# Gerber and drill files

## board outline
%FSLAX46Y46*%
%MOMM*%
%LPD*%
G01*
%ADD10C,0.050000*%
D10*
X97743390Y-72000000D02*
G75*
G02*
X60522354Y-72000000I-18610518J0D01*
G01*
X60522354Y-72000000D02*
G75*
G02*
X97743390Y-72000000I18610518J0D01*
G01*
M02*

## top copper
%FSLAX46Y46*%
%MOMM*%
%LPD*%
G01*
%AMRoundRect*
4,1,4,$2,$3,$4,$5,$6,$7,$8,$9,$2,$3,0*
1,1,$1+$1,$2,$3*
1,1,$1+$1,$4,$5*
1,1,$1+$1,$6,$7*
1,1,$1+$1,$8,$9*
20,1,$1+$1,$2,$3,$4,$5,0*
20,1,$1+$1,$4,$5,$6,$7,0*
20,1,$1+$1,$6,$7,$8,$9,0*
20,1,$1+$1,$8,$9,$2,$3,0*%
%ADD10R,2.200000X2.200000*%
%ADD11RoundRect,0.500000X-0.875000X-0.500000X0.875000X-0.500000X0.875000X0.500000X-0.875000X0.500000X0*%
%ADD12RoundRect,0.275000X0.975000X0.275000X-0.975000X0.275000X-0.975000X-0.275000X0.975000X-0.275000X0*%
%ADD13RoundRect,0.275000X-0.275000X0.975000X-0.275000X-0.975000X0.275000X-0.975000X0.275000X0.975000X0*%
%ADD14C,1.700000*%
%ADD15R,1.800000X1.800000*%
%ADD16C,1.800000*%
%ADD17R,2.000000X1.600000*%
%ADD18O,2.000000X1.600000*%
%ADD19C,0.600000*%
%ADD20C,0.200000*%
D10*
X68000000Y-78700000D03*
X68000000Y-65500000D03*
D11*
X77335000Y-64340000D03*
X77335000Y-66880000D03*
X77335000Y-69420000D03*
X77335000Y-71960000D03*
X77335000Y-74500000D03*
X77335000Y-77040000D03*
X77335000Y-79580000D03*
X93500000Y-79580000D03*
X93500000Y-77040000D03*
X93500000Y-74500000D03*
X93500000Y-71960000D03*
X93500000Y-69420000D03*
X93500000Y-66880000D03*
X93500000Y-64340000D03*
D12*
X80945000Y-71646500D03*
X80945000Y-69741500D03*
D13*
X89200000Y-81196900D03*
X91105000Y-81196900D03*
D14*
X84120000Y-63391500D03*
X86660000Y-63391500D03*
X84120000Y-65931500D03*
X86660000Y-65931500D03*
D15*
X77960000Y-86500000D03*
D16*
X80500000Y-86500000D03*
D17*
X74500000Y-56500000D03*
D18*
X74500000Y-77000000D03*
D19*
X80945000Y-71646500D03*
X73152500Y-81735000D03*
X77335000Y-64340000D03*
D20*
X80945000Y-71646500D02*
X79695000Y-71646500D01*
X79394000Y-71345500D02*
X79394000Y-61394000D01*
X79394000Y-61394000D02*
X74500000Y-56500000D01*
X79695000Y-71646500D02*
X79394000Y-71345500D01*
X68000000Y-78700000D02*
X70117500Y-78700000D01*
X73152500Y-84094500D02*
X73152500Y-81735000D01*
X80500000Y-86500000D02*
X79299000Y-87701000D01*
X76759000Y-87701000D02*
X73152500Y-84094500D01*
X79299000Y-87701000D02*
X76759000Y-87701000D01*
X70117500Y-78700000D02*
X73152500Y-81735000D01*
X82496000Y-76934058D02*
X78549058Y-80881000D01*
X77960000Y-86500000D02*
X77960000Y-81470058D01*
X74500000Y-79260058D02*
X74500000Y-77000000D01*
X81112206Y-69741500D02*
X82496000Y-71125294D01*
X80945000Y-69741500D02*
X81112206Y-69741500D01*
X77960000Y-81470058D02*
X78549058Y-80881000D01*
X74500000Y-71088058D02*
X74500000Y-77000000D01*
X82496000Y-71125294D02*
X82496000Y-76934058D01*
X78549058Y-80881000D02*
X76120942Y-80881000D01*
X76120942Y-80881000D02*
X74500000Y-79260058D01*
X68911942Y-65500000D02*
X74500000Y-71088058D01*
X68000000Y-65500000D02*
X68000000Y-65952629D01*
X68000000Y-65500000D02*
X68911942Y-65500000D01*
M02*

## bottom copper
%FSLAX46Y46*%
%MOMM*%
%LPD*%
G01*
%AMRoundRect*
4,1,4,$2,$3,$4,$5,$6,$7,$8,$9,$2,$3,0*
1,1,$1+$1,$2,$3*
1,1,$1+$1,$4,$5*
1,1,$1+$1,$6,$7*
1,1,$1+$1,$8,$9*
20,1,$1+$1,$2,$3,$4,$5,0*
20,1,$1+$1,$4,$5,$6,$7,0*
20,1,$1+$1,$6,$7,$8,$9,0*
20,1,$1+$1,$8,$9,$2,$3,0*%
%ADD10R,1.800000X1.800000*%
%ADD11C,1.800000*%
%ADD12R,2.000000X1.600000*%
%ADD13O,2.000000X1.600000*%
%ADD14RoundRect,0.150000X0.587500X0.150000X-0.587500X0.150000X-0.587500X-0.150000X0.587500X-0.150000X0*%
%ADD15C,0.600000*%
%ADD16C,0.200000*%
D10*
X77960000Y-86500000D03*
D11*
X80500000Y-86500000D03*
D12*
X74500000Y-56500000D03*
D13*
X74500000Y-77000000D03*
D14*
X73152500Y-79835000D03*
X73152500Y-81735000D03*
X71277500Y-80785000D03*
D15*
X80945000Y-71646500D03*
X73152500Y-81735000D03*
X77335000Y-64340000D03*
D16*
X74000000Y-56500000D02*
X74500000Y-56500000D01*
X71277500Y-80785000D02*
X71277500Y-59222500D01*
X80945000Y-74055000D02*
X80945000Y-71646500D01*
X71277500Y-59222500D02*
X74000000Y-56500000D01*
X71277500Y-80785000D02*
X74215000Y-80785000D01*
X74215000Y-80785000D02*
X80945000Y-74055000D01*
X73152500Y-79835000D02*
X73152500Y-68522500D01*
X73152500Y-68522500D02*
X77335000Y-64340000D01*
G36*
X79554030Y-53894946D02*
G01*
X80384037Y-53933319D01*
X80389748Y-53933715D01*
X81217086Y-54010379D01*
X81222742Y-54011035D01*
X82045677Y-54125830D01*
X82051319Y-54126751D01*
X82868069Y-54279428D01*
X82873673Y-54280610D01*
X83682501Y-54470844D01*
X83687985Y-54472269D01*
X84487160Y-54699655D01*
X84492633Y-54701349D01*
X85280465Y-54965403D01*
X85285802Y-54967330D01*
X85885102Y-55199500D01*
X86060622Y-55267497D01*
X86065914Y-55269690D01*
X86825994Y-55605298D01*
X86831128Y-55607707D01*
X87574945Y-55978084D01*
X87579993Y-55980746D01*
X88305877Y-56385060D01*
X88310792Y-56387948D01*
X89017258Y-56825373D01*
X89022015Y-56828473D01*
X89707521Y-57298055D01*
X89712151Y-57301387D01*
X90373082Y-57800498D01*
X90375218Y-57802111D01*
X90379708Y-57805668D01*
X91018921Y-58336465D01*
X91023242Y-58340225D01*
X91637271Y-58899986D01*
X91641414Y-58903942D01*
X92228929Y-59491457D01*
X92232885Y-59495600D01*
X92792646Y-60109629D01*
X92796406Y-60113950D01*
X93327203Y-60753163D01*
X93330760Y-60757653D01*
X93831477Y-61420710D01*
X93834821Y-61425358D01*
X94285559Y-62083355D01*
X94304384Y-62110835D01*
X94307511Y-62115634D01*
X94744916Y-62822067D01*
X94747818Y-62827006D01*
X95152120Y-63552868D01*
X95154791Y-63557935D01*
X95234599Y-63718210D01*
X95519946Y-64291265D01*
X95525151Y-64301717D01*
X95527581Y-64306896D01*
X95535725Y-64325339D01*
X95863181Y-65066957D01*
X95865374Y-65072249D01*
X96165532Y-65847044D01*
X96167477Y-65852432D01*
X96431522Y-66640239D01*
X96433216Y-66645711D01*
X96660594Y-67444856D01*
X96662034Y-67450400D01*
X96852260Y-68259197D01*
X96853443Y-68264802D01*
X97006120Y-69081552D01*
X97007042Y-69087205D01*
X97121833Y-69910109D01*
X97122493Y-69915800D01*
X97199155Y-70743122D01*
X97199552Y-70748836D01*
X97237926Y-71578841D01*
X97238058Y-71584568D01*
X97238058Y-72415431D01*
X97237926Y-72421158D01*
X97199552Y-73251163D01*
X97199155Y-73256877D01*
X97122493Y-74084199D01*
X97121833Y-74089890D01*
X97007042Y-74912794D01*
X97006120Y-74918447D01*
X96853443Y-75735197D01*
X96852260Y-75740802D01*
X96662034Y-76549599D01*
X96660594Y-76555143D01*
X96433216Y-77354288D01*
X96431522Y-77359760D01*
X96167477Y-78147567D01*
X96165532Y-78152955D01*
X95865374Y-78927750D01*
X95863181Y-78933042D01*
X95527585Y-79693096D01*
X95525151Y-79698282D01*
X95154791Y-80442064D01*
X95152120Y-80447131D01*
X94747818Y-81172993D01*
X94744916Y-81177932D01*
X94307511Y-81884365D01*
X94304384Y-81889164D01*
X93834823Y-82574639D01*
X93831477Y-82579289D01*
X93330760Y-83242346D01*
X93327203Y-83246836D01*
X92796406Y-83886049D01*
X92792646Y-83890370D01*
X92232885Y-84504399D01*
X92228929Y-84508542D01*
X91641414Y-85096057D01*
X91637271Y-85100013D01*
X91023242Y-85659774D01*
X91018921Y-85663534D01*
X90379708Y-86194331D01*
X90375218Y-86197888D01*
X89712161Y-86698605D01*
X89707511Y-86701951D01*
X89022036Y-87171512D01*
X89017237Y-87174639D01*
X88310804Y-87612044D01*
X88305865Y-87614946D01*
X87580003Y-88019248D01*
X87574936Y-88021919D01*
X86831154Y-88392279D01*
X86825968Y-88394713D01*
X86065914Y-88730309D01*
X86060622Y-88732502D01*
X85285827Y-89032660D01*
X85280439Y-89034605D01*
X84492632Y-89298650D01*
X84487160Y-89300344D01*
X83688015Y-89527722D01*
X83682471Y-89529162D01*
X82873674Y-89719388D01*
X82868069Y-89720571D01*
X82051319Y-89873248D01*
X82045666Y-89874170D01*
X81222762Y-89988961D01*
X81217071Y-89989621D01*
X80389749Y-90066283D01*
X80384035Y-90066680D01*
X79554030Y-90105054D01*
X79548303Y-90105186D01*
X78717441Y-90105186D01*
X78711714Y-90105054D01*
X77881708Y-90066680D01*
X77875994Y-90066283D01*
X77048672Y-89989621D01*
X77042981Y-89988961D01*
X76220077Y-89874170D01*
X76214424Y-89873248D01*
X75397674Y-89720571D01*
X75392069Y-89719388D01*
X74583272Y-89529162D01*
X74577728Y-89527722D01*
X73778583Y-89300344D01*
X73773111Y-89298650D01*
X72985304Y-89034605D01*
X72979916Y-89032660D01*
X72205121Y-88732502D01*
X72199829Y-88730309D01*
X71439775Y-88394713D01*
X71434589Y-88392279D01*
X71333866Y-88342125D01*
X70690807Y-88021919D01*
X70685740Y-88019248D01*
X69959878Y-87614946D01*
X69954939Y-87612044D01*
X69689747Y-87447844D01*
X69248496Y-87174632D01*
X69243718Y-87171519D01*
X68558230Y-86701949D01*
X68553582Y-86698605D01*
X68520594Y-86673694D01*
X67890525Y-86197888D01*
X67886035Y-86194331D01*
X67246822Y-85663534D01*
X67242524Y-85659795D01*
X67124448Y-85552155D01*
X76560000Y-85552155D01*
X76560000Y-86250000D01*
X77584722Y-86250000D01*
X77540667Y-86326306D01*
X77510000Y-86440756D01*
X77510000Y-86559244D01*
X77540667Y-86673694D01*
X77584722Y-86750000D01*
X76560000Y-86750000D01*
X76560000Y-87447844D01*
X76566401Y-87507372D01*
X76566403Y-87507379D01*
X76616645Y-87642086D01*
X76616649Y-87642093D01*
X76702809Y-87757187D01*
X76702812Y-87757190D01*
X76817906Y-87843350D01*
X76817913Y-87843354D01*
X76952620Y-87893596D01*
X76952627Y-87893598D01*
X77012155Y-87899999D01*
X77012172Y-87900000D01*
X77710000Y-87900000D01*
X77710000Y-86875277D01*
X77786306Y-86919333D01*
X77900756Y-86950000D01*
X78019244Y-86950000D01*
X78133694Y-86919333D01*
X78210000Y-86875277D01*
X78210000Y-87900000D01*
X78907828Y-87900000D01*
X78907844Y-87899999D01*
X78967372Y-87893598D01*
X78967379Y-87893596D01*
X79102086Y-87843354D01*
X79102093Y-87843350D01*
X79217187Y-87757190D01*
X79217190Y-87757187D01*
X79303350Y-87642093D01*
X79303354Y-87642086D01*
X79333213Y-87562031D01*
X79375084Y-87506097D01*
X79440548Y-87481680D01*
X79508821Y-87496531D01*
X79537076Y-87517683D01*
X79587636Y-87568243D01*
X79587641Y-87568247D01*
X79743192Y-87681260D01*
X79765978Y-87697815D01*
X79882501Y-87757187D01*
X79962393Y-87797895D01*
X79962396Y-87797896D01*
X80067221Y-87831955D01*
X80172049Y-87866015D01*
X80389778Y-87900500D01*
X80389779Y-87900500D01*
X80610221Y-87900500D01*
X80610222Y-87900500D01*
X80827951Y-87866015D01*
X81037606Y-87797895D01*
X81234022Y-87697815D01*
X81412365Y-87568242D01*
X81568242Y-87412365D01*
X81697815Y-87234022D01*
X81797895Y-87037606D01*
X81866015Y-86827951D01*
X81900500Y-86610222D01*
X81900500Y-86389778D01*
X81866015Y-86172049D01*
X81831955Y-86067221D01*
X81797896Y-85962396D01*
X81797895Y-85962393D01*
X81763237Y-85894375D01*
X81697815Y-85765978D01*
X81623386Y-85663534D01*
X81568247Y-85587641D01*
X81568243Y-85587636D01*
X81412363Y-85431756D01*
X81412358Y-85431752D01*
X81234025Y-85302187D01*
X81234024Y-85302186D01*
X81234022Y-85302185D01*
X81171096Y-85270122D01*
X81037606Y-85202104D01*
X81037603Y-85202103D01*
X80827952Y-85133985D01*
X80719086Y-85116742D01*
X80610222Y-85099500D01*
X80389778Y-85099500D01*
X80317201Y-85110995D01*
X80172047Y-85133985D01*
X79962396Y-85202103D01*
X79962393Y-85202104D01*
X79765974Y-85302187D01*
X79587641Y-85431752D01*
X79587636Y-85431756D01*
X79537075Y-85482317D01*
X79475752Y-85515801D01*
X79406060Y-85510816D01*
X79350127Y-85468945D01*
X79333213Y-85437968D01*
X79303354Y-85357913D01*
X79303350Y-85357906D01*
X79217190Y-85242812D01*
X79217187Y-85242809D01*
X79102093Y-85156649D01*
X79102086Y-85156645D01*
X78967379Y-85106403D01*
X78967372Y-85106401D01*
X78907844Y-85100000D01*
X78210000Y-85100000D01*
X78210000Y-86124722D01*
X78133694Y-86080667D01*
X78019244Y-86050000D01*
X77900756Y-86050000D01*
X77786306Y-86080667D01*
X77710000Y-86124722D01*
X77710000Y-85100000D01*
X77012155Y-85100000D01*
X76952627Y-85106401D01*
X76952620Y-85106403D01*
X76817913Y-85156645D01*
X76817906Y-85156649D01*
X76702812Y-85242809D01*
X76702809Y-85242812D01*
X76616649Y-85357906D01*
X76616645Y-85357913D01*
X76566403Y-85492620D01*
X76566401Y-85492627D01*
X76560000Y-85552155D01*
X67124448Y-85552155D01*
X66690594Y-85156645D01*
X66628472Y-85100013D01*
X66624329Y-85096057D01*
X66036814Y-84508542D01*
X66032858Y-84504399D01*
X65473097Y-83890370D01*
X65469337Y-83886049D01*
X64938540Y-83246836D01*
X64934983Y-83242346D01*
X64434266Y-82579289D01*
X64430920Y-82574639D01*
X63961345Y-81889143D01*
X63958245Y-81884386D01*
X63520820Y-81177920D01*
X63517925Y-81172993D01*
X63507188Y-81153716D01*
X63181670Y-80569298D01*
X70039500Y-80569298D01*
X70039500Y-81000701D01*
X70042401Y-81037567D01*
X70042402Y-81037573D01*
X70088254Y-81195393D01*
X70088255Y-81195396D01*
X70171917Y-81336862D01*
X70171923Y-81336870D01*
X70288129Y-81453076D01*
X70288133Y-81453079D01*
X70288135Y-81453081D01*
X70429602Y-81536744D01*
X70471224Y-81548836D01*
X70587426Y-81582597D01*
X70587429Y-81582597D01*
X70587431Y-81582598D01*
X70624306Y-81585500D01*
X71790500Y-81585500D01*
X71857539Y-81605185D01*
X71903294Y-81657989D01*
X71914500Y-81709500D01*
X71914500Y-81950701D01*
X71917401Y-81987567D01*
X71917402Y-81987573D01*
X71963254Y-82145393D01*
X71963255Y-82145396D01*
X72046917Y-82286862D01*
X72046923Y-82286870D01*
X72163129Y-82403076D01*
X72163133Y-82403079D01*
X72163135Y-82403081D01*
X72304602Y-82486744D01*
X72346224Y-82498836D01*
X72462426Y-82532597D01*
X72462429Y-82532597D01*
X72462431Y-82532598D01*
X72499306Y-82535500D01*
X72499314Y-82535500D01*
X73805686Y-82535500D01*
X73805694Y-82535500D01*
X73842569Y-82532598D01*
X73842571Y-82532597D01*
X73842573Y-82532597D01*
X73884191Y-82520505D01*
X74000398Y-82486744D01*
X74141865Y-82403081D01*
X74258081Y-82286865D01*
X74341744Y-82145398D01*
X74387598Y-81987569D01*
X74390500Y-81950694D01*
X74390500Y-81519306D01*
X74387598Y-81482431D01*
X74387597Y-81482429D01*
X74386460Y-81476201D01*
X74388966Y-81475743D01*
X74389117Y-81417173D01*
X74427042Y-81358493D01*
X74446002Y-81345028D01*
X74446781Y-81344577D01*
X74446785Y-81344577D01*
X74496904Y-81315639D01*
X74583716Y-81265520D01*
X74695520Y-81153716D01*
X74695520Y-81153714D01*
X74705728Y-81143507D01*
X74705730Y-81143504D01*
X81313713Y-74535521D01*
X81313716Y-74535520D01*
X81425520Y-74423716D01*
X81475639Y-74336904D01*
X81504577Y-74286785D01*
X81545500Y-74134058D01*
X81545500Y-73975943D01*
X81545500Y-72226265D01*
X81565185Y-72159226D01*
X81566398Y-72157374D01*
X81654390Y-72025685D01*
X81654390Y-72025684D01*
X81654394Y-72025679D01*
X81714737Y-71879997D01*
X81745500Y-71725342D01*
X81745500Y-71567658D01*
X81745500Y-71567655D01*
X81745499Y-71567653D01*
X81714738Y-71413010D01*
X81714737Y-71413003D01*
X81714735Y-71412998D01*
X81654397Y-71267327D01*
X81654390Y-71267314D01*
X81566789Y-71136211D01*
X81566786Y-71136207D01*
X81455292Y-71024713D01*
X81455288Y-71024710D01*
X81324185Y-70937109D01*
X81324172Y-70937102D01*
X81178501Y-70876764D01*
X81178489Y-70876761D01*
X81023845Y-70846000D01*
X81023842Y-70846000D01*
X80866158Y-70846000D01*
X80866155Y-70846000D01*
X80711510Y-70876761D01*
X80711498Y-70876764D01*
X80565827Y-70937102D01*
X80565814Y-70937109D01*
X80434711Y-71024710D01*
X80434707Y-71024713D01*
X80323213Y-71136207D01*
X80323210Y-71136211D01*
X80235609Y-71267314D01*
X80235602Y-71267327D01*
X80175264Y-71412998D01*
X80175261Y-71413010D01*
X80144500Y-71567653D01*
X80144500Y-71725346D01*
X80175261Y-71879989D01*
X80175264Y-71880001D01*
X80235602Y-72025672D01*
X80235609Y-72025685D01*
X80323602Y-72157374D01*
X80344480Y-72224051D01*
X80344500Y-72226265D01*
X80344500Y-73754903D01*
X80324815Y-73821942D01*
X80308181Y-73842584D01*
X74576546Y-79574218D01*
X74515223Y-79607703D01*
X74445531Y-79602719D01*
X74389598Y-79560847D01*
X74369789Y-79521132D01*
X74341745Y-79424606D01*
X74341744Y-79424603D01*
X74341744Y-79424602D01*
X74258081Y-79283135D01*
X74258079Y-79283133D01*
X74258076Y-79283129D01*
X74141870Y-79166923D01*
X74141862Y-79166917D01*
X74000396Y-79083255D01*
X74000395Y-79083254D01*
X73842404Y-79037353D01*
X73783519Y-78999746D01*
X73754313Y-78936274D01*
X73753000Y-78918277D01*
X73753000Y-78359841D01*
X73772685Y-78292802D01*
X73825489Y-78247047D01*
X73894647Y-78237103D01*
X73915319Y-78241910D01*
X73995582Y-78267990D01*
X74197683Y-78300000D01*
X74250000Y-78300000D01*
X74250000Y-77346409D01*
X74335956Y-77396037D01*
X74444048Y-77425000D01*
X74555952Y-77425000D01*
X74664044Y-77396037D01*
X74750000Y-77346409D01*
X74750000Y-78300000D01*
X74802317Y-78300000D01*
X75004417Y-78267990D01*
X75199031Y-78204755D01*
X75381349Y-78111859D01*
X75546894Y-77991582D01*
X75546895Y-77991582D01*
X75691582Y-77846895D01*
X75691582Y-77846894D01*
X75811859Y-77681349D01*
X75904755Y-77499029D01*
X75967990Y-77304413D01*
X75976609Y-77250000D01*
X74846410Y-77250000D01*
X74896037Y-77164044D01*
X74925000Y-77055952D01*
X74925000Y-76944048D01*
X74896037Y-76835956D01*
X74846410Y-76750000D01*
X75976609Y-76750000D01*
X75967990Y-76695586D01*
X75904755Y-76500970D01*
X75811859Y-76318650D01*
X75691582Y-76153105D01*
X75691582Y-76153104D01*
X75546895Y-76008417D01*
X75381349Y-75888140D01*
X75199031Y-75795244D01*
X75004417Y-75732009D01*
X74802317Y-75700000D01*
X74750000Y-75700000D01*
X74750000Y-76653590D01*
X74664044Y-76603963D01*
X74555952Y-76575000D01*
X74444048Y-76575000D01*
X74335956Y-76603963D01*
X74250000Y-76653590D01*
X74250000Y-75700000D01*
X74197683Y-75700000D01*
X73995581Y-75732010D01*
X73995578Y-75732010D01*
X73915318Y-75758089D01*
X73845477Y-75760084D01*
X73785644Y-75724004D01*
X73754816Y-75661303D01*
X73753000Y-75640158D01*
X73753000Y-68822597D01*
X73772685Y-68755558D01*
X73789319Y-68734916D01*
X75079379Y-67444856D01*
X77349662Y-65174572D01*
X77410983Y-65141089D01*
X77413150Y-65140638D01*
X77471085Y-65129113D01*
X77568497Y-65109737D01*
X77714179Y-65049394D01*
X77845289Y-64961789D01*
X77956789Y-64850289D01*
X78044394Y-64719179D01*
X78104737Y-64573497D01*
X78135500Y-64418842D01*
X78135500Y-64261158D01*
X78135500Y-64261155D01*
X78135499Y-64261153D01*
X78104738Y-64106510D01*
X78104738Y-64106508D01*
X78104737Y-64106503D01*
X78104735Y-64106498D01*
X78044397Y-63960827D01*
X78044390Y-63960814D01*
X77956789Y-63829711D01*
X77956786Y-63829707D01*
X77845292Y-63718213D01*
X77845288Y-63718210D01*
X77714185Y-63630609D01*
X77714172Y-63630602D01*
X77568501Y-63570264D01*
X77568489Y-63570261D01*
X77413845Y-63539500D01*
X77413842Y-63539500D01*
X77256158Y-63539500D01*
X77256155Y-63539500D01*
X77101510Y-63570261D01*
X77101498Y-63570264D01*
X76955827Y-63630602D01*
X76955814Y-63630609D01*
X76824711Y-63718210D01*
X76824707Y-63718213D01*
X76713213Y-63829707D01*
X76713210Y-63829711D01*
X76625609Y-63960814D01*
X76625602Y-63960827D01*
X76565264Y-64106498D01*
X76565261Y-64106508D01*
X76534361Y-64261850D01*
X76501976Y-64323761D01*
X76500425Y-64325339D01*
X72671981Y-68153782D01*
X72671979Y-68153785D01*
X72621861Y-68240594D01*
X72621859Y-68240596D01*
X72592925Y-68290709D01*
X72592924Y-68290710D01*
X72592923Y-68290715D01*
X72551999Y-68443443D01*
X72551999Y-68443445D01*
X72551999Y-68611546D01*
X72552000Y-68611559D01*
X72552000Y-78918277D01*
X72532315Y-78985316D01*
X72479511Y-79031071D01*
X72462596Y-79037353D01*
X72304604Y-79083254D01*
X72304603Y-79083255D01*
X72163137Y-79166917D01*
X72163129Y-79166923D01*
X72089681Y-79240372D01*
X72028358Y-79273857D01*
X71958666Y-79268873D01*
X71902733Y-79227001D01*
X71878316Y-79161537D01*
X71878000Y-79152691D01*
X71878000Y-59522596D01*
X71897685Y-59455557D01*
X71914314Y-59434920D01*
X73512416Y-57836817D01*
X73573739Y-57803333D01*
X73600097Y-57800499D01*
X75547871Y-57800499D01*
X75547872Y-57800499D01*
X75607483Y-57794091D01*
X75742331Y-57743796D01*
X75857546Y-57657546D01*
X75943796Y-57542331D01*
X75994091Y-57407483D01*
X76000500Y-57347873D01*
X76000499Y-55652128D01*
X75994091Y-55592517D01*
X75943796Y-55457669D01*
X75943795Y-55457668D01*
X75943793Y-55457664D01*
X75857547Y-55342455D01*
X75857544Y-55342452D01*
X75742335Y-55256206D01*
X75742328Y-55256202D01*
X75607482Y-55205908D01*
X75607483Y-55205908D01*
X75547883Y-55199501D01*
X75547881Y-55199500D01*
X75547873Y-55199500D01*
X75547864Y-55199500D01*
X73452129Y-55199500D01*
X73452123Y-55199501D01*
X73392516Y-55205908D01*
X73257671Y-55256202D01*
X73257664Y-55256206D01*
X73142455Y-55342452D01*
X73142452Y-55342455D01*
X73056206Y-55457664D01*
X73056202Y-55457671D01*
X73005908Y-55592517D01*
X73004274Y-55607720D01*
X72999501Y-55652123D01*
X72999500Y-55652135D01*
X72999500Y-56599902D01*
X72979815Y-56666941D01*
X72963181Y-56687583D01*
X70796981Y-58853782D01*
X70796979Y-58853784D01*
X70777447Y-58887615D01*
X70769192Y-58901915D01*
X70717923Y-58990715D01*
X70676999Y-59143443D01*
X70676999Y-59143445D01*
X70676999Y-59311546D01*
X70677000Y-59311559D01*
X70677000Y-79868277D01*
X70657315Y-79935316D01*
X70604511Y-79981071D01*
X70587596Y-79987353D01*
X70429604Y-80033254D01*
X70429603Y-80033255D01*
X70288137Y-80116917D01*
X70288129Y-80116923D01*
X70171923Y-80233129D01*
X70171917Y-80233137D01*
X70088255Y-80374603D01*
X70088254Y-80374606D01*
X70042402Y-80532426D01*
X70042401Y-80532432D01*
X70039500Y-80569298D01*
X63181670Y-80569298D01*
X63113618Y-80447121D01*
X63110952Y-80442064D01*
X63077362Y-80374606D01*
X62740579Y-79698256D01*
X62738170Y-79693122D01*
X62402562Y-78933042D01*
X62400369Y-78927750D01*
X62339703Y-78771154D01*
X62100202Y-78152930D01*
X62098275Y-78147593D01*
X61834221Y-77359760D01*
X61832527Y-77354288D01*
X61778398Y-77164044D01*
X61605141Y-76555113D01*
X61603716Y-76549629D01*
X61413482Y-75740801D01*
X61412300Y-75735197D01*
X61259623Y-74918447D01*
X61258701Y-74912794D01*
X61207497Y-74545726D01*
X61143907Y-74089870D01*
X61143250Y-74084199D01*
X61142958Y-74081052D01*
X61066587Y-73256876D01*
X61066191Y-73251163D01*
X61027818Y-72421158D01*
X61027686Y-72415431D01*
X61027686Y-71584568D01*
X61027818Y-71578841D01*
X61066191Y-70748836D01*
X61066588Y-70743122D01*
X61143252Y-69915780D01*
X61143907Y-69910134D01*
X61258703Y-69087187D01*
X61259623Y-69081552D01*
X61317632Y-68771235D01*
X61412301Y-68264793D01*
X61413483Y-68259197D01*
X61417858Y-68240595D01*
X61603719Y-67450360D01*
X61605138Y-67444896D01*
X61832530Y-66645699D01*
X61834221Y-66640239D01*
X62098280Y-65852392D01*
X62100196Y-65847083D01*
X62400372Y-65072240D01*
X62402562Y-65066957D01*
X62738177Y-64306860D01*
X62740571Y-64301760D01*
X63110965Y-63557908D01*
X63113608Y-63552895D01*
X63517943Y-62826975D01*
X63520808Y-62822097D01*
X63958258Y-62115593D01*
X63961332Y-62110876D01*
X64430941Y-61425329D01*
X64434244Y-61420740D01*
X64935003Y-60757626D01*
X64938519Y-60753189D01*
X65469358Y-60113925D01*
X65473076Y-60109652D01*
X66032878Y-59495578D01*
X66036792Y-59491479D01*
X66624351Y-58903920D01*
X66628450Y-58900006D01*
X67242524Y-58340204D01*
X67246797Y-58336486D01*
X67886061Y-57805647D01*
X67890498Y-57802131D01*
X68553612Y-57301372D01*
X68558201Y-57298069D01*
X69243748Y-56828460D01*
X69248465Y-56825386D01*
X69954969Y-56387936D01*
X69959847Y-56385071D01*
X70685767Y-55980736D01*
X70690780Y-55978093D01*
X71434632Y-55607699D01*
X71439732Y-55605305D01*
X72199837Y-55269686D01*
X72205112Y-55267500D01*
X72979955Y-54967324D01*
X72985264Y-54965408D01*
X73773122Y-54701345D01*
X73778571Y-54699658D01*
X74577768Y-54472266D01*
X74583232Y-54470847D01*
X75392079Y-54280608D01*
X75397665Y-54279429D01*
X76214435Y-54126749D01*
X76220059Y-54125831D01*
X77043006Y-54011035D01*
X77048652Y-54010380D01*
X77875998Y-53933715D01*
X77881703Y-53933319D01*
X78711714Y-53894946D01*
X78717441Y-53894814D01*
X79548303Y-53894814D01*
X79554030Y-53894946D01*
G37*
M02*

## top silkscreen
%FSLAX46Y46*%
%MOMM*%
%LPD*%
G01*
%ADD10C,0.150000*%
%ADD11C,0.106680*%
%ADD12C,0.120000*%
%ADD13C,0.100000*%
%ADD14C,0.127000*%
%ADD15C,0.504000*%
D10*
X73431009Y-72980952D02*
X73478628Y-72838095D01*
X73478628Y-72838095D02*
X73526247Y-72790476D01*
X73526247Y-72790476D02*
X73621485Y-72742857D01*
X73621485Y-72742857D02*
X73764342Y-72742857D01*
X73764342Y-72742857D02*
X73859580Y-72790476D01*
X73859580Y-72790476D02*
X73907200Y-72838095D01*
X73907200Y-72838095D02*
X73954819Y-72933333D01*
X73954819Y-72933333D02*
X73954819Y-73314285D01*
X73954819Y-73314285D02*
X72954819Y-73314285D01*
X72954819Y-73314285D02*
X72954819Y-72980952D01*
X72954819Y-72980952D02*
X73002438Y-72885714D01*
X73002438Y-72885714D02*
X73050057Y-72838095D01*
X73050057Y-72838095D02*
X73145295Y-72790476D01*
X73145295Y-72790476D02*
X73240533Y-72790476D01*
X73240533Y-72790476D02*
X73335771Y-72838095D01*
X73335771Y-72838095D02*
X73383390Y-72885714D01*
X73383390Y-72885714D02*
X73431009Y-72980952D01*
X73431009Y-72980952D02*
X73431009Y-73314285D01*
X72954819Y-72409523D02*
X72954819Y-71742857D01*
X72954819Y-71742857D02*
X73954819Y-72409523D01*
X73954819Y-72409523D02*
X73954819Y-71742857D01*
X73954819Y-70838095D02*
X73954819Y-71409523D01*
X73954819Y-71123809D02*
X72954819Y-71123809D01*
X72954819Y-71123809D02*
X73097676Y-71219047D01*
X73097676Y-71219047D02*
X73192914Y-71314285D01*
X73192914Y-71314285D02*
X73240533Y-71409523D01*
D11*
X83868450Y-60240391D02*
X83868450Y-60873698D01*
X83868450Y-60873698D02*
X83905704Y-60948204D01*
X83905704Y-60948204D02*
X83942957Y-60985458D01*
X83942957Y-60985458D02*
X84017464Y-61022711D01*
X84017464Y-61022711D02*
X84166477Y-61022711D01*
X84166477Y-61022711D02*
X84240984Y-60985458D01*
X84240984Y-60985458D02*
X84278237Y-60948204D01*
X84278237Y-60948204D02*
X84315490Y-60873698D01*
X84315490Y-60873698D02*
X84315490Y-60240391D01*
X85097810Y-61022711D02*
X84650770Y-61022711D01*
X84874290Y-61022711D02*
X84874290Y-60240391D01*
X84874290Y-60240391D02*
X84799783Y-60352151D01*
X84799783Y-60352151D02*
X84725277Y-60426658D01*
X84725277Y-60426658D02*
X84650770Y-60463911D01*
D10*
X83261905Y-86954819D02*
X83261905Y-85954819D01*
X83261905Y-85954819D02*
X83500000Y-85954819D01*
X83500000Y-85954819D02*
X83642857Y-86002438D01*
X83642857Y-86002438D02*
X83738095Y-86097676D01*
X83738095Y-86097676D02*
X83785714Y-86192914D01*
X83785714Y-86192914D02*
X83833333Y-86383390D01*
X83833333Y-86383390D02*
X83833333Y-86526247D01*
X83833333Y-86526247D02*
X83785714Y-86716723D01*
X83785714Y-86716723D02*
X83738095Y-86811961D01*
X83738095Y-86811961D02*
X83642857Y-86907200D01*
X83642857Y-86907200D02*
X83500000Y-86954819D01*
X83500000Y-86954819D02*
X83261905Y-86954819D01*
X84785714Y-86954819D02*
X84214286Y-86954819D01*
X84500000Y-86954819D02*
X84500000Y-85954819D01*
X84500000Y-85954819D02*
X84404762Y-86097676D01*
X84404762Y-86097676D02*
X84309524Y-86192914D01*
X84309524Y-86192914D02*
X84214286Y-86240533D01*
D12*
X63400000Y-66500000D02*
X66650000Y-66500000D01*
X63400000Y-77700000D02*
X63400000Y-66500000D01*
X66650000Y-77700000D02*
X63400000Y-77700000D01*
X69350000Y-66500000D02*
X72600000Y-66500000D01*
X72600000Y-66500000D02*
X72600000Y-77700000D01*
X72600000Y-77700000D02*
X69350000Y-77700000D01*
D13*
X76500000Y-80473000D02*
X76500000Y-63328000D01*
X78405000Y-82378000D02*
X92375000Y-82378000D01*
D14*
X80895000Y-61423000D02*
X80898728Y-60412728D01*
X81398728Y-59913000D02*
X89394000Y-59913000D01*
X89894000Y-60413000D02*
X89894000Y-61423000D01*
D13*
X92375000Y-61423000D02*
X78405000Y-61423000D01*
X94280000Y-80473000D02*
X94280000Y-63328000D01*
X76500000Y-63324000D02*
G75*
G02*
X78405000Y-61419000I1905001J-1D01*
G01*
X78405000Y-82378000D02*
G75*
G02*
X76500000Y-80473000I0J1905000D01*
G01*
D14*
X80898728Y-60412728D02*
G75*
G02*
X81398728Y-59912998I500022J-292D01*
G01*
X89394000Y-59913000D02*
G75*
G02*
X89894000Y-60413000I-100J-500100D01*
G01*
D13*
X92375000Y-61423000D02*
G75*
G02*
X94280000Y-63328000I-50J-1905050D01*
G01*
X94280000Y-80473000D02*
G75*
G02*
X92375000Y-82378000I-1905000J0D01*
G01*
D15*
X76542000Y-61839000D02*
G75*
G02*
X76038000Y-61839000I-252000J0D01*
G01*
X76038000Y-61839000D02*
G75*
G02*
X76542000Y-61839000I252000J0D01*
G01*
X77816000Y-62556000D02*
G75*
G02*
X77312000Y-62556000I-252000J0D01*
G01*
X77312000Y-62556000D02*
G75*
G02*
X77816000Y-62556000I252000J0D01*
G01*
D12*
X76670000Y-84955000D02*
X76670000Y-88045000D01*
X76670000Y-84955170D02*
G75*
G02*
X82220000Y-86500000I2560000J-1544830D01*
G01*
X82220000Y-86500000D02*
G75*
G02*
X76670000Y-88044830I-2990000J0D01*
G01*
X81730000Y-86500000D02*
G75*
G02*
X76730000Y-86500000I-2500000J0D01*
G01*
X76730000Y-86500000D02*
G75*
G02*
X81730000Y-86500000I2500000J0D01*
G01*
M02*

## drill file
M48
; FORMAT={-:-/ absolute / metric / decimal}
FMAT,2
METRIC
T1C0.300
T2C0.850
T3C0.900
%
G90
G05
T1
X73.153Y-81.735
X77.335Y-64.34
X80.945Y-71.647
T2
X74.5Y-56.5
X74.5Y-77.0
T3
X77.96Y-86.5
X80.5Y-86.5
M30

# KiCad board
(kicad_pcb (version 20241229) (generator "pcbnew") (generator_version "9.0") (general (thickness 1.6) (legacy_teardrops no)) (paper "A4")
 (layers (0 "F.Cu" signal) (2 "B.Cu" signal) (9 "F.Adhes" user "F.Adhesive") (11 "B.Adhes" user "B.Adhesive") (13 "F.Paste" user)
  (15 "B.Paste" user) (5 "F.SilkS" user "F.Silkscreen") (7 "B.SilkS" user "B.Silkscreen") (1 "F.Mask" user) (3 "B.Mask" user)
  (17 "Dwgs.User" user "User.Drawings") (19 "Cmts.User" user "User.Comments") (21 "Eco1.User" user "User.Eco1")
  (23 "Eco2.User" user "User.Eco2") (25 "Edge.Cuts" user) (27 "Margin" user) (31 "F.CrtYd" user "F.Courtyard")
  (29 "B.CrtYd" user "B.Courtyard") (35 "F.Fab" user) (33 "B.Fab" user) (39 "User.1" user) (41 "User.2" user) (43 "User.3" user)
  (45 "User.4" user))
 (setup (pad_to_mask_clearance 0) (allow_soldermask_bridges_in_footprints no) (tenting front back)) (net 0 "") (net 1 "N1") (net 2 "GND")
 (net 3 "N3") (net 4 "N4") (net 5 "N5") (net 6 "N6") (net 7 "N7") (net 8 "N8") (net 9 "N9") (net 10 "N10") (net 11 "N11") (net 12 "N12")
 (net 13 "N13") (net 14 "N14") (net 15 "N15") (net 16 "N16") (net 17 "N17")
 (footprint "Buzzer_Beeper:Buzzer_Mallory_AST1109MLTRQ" (layer "F.Cu") (at 68 72.1 90)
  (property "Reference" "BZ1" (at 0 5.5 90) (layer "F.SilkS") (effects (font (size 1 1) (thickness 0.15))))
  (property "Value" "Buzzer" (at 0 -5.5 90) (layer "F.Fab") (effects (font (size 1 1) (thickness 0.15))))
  (fp_line (start 5.6 -4.6) (end 5.6 -1.35) (stroke (width 0.12) (type solid)) (layer "F.SilkS"))
  (fp_line (start -5.6 -4.6) (end 5.6 -4.6) (stroke (width 0.12) (type solid)) (layer "F.SilkS"))
  (fp_line (start -5.6 -1.35) (end -5.6 -4.6) (stroke (width 0.12) (type solid)) (layer "F.SilkS"))
  (fp_line (start 5.6 1.35) (end 5.6 4.6) (stroke (width 0.12) (type solid)) (layer "F.SilkS"))
  (fp_line (start 5.6 4.6) (end -5.6 4.6) (stroke (width 0.12) (type solid)) (layer "F.SilkS"))
  (fp_line (start -5.6 4.6) (end -5.6 1.35) (stroke (width 0.12) (type solid)) (layer "F.SilkS"))
  (pad "1" smd rect (at -6.6 0 90) (size 2.2 2.2) (layers "F.Cu" "F.Mask" "F.Paste") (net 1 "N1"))
  (pad "2" smd rect (at 6.6 0 90) (size 2.2 2.2) (layers "F.Cu" "F.Mask" "F.Paste") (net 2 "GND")))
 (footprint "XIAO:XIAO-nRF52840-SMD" (layer "F.Cu") (at 76.5 82.46)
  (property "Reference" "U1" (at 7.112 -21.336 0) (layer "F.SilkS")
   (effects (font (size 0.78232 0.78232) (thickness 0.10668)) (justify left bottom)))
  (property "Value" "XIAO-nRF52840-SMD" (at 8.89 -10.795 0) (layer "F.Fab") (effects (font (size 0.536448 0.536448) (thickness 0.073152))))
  (fp_line (start 0 -1.987) (end 0 -19.132) (stroke (width 0.1) (type solid)) (layer "F.SilkS"))
  (fp_line (start 1.905 -0.082) (end 15.875 -0.082) (stroke (width 0.1) (type solid)) (layer "F.SilkS"))
  (fp_line (start 4.395 -21.037) (end 4.398728 -22.047272) (stroke (width 0.127) (type solid)) (layer "F.SilkS"))
  (fp_line (start 4.898728 -22.547) (end 12.894 -22.547) (stroke (width 0.127) (type solid)) (layer "F.SilkS"))
  (fp_line (start 13.394 -22.047) (end 13.394 -21.037) (stroke (width 0.127) (type solid)) (layer "F.SilkS"))
  (fp_line (start 15.875 -21.037) (end 1.905 -21.037) (stroke (width 0.1) (type solid)) (layer "F.SilkS"))
  (fp_line (start 17.78 -1.987) (end 17.78 -19.132) (stroke (width 0.1) (type solid)) (layer "F.SilkS"))
  (fp_arc (start 0 -19.136) (mid 0.557962 -20.483038) (end 1.905 -21.041) (stroke (width 0.1) (type solid)) (layer "F.SilkS"))
  (fp_arc (start 1.905 -0.082) (mid 0.557962 -0.639962) (end 0 -1.987) (stroke (width 0.1) (type solid)) (layer "F.SilkS"))
  (fp_arc (start 4.398728 -22.047272) (mid 4.545276 -22.400644) (end 4.898728 -22.547) (stroke (width 0.127) (type default))
   (layer "F.SilkS"))
  (fp_arc (start 12.894 -22.547) (mid 13.247531 -22.400546) (end 13.394 -22.047) (stroke (width 0.127) (type default)) (layer "F.SilkS"))
  (fp_arc (start 15.875 -21.037) (mid 17.222016 -20.479031) (end 17.78 -19.132) (stroke (width 0.1) (type solid)) (layer "F.SilkS"))
  (fp_arc (start 17.78 -1.987) (mid 17.222038 -0.639961) (end 15.875 -0.082) (stroke (width 0.1) (type solid)) (layer "F.SilkS"))
  (fp_circle (center -0.21 -20.621) (end -0.21 -20.875) (stroke (width 0.5) (type solid)) (fill yes) (layer "F.SilkS"))
  (fp_circle (center 1.064 -19.904) (end 1.064 -20.158) (stroke (width 0.5) (type solid)) (fill yes) (layer "F.SilkS"))
  (pad "1" smd roundrect (at 0.835 -18.12) (size 2.75 2) (layers "F.Cu" "F.Mask" "F.Paste") (roundrect_rratio 0.25) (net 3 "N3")
   (solder_mask_margin 0.0508) (thermal_bridge_angle 45))
  (pad "2" smd roundrect (at 0.835 -15.58) (size 2.75 2) (layers "F.Cu" "F.Mask" "F.Paste") (roundrect_rratio 0.25) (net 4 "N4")
   (solder_mask_margin 0.0508) (thermal_bridge_angle 45))
  (pad "3" smd roundrect (at 0.835 -13.04) (size 2.75 2) (layers "F.Cu" "F.Mask" "F.Paste") (roundrect_rratio 0.25) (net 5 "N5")
   (solder_mask_margin 0.0508) (thermal_bridge_angle 45))
  (pad "4" smd roundrect (at 0.835 -10.5) (size 2.75 2) (layers "F.Cu" "F.Mask" "F.Paste") (roundrect_rratio 0.25) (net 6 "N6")
   (solder_mask_margin 0.0508) (thermal_bridge_angle 45))
  (pad "5" smd roundrect (at 0.835 -7.96) (size 2.75 2) (layers "F.Cu" "F.Mask" "F.Paste") (roundrect_rratio 0.25) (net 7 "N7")
   (solder_mask_margin 0.0508) (thermal_bridge_angle 45))
  (pad "6" smd roundrect (at 0.835 -5.42) (size 2.75 2) (layers "F.Cu" "F.Mask" "F.Paste") (roundrect_rratio 0.25) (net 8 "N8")
   (solder_mask_margin 0.0508) (thermal_bridge_angle 45))
  (pad "7" smd roundrect (at 0.835 -2.88) (size 2.75 2) (layers "F.Cu" "F.Mask" "F.Paste") (roundrect_rratio 0.25) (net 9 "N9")
   (solder_mask_margin 0.0508) (thermal_bridge_angle 45))
  (pad "8" smd roundrect (at 17 -2.88) (size 2.75 2) (layers "F.Cu" "F.Mask" "F.Paste") (roundrect_rratio 0.25) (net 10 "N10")
   (solder_mask_margin 0.0508) (thermal_bridge_angle 45))
  (pad "9" smd roundrect (at 17 -5.42) (size 2.75 2) (layers "F.Cu" "F.Mask" "F.Paste") (roundrect_rratio 0.25) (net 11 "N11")
   (solder_mask_margin 0.0508) (thermal_bridge_angle 45))
  (pad "10" smd roundrect (at 17 -7.96) (size 2.75 2) (layers "F.Cu" "F.Mask" "F.Paste") (roundrect_rratio 0.25) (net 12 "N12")
   (solder_mask_margin 0.0508) (thermal_bridge_angle 45))
  (pad "11" smd roundrect (at 17 -10.5) (size 2.75 2) (layers "F.Cu" "F.Mask" "F.Paste") (roundrect_rratio 0.25) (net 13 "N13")
   (solder_mask_margin 0.0508) (thermal_bridge_angle 45))
  (pad "12" smd roundrect (at 17 -13.04) (size 2.75 2) (layers "F.Cu" "F.Mask" "F.Paste") (roundrect_rratio 0.25) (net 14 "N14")
   (solder_mask_margin 0.0508) (thermal_bridge_angle 45))
  (pad "13" smd roundrect (at 17 -15.58) (size 2.75 2) (layers "F.Cu" "F.Mask" "F.Paste") (roundrect_rratio 0.25) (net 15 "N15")
   (solder_mask_margin 0.0508) (thermal_bridge_angle 45))
  (pad "14" smd roundrect (at 17 -18.12) (size 2.75 2) (layers "F.Cu" "F.Mask" "F.Paste") (roundrect_rratio 0.25) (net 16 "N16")
   (solder_mask_margin 0.0508) (thermal_bridge_angle 45))
  (pad "15" smd roundrect (at 4.445 -10.8135 180) (size 2.5 1.1) (layers "F.Cu" "F.Mask" "F.Paste") (roundrect_rratio 0.25) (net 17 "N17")
   (solder_mask_margin 0.0508) (thermal_bridge_angle 45))
  (pad "16" smd roundrect (at 4.445 -12.7185 180) (size 2.5 1.1) (layers "F.Cu" "F.Mask" "F.Paste") (roundrect_rratio 0.25) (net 2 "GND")
   (solder_mask_margin 0.0508) (thermal_bridge_angle 45))
  (pad "17" smd roundrect (at 12.7 -1.2631 270) (size 2.5 1.1) (layers "F.Cu" "F.Mask" "F.Paste") (roundrect_rratio 0.25)
   (solder_mask_margin 0.0508) (thermal_bridge_angle 45))
  (pad "18" smd roundrect (at 14.605 -1.2631 270) (size 2.5 1.1) (layers "F.Cu" "F.Mask" "F.Paste") (roundrect_rratio 0.25)
   (solder_mask_margin 0.0508) (thermal_bridge_angle 45))
  (pad "19" smd circle (at 7.62 -19.0685) (size 1.7 1.7) (layers "F.Cu" "F.Mask" "F.Paste"))
  (pad "20" smd circle (at 10.16 -19.0685) (size 1.7 1.7) (layers "F.Cu" "F.Mask" "F.Paste"))
  (pad "21" smd circle (at 7.62 -16.5285) (size 1.7 1.7) (layers "F.Cu" "F.Mask" "F.Paste"))
  (pad "22" smd circle (at 10.16 -16.5285) (size 1.7 1.7) (layers "F.Cu" "F.Mask" "F.Paste")))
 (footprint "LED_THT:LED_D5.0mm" (layer "F.Cu") (at 77.96 86.5)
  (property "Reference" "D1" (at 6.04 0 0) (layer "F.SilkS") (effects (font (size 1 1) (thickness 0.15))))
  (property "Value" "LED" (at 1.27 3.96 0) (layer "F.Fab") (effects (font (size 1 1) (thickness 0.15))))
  (fp_line (start -1.29 -1.545) (end -1.29 1.545) (stroke (width 0.12) (type solid)) (layer "F.SilkS"))
  (fp_arc (start -1.29 -1.54483) (mid 2.071779 -2.880495) (end 4.26 0) (stroke (width 0.12) (type solid)) (layer "F.SilkS"))
  (fp_arc (start 4.26 0) (mid 2.071779 2.880495) (end -1.29 1.54483) (stroke (width 0.12) (type solid)) (layer "F.SilkS"))
  (fp_circle (center 1.27 0) (end 3.77 0) (stroke (width 0.12) (type solid)) (fill no) (layer "F.SilkS"))
  (pad "1" thru_hole rect (at 0 0) (size 1.8 1.8) (drill 0.9) (layers "*.Cu" "*.Mask") (remove_unused_layers no) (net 2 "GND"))
  (pad "2" thru_hole circle (at 2.54 0) (size 1.8 1.8) (drill 0.9) (layers "*.Cu" "*.Mask") (remove_unused_layers no) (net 1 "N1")))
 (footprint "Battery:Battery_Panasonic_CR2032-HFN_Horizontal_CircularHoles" (layer "B.Cu") (at 74.5 56.5 -90)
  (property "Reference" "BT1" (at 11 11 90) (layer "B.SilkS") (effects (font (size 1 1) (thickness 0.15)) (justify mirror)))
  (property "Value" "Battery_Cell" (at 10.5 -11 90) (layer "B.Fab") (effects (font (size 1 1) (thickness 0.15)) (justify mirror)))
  (pad "1" thru_hole rect (at 0 0 270) (size 1.6 2) (drill 0.85) (layers "*.Cu" "*.Mask") (remove_unused_layers no) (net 17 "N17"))
  (pad "2" thru_hole oval (at 20.5 0 270) (size 1.6 2) (drill 0.85) (layers "*.Cu" "*.Mask") (remove_unused_layers no) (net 2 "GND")))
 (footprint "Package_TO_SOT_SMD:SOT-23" (layer "B.Cu") (at 72.215 80.785 180)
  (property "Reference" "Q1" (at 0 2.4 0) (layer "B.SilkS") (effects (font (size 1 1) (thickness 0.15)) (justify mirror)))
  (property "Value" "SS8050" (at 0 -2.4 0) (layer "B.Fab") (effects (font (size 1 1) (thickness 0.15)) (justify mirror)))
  (pad "1" smd roundrect (at -0.9375 0.95 180) (size 1.475 0.6) (layers "B.Cu" "B.Mask" "B.Paste") (roundrect_rratio 0.25) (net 3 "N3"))
  (pad "2" smd roundrect (at -0.9375 -0.95 180) (size 1.475 0.6) (layers "B.Cu" "B.Mask" "B.Paste") (roundrect_rratio 0.25) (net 1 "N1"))
  (pad "3" smd roundrect (at 0.9375 0 180) (size 1.475 0.6) (layers "B.Cu" "B.Mask" "B.Paste") (roundrect_rratio 0.25) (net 17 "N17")))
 (gr_circle (center 79.132872 72) (end 97.5 69) (stroke (width 0.05) (type default)) (fill no) (layer "Edge.Cuts"))
 (segment (start 80.945 71.6465) (end 79.695 71.6465) (width 0.2) (layer "F.Cu") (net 17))
 (segment (start 79.394 71.3455) (end 79.394 61.394) (width 0.2) (layer "F.Cu") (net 17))
 (segment (start 79.394 61.394) (end 74.5 56.5) (width 0.2) (layer "F.Cu") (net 17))
 (segment (start 79.695 71.6465) (end 79.394 71.3455) (width 0.2) (layer "F.Cu") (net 17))
 (via (at 80.945 71.6465) (size 0.6) (drill 0.3) (layers "F.Cu" "B.Cu") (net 17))
 (segment (start 74 56.5) (end 74.5 56.5) (width 0.2) (layer "B.Cu") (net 17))
 (segment (start 71.2775 80.785) (end 71.2775 59.2225) (width 0.2) (layer "B.Cu") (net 17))
 (segment (start 80.945 74.055) (end 80.945 71.6465) (width 0.2) (layer "B.Cu") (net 17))
 (segment (start 71.2775 59.2225) (end 74 56.5) (width 0.2) (layer "B.Cu") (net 17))
 (segment (start 71.2775 80.785) (end 74.215 80.785) (width 0.2) (layer "B.Cu") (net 17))
 (segment (start 74.215 80.785) (end 80.945 74.055) (width 0.2) (layer "B.Cu") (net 17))
 (segment (start 68 78.7) (end 70.1175 78.7) (width 0.2) (layer "F.Cu") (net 1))
 (segment (start 73.1525 84.0945) (end 73.1525 81.735) (width 0.2) (layer "F.Cu") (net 1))
 (segment (start 80.5 86.5) (end 79.299 87.701) (width 0.2) (layer "F.Cu") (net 1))
 (segment (start 76.759 87.701) (end 73.1525 84.0945) (width 0.2) (layer "F.Cu") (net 1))
 (segment (start 79.299 87.701) (end 76.759 87.701) (width 0.2) (layer "F.Cu") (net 1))
 (segment (start 70.1175 78.7) (end 73.1525 81.735) (width 0.2) (layer "F.Cu") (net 1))
 (via (at 73.1525 81.735) (size 0.6) (drill 0.3) (layers "F.Cu" "B.Cu") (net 1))
 (via (at 77.335 64.34) (size 0.6) (drill 0.3) (layers "F.Cu" "B.Cu") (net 3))
 (segment (start 73.1525 79.835) (end 73.1525 68.5225) (width 0.2) (layer "B.Cu") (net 3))
 (segment (start 73.1525 68.5225) (end 77.335 64.34) (width 0.2) (layer "B.Cu") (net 3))
 (segment (start 82.496 76.934058) (end 78.549058 80.881) (width 0.2) (layer "F.Cu") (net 2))
 (segment (start 77.96 86.5) (end 77.96 81.470058) (width 0.2) (layer "F.Cu") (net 2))
 (segment (start 74.5 79.260058) (end 74.5 77) (width 0.2) (layer "F.Cu") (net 2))
 (segment (start 81.112206 69.7415) (end 82.496 71.125294) (width 0.2) (layer "F.Cu") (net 2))
 (segment (start 80.945 69.7415) (end 81.112206 69.7415) (width 0.2) (layer "F.Cu") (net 2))
 (segment (start 77.96 81.470058) (end 78.549058 80.881) (width 0.2) (layer "F.Cu") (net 2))
 (segment (start 74.5 71.088058) (end 74.5 77) (width 0.2) (layer "F.Cu") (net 2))
 (segment (start 82.496 71.125294) (end 82.496 76.934058) (width 0.2) (layer "F.Cu") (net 2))
 (segment (start 78.549058 80.881) (end 76.120942 80.881) (width 0.2) (layer "F.Cu") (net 2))
 (segment (start 76.120942 80.881) (end 74.5 79.260058) (width 0.2) (layer "F.Cu") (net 2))
 (segment (start 68.911942 65.5) (end 74.5 71.088058) (width 0.2) (layer "F.Cu") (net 2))
 (segment (start 68 65.5) (end 68 65.952629) (width 0.2) (layer "F.Cu") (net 2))
 (segment (start 68 65.5) (end 68.911942 65.5) (width 0.2) (layer "F.Cu") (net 2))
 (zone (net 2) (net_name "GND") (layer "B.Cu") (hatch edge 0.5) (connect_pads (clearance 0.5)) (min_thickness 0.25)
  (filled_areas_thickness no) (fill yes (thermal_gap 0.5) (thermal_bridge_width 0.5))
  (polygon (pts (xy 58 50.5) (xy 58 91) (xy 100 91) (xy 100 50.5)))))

